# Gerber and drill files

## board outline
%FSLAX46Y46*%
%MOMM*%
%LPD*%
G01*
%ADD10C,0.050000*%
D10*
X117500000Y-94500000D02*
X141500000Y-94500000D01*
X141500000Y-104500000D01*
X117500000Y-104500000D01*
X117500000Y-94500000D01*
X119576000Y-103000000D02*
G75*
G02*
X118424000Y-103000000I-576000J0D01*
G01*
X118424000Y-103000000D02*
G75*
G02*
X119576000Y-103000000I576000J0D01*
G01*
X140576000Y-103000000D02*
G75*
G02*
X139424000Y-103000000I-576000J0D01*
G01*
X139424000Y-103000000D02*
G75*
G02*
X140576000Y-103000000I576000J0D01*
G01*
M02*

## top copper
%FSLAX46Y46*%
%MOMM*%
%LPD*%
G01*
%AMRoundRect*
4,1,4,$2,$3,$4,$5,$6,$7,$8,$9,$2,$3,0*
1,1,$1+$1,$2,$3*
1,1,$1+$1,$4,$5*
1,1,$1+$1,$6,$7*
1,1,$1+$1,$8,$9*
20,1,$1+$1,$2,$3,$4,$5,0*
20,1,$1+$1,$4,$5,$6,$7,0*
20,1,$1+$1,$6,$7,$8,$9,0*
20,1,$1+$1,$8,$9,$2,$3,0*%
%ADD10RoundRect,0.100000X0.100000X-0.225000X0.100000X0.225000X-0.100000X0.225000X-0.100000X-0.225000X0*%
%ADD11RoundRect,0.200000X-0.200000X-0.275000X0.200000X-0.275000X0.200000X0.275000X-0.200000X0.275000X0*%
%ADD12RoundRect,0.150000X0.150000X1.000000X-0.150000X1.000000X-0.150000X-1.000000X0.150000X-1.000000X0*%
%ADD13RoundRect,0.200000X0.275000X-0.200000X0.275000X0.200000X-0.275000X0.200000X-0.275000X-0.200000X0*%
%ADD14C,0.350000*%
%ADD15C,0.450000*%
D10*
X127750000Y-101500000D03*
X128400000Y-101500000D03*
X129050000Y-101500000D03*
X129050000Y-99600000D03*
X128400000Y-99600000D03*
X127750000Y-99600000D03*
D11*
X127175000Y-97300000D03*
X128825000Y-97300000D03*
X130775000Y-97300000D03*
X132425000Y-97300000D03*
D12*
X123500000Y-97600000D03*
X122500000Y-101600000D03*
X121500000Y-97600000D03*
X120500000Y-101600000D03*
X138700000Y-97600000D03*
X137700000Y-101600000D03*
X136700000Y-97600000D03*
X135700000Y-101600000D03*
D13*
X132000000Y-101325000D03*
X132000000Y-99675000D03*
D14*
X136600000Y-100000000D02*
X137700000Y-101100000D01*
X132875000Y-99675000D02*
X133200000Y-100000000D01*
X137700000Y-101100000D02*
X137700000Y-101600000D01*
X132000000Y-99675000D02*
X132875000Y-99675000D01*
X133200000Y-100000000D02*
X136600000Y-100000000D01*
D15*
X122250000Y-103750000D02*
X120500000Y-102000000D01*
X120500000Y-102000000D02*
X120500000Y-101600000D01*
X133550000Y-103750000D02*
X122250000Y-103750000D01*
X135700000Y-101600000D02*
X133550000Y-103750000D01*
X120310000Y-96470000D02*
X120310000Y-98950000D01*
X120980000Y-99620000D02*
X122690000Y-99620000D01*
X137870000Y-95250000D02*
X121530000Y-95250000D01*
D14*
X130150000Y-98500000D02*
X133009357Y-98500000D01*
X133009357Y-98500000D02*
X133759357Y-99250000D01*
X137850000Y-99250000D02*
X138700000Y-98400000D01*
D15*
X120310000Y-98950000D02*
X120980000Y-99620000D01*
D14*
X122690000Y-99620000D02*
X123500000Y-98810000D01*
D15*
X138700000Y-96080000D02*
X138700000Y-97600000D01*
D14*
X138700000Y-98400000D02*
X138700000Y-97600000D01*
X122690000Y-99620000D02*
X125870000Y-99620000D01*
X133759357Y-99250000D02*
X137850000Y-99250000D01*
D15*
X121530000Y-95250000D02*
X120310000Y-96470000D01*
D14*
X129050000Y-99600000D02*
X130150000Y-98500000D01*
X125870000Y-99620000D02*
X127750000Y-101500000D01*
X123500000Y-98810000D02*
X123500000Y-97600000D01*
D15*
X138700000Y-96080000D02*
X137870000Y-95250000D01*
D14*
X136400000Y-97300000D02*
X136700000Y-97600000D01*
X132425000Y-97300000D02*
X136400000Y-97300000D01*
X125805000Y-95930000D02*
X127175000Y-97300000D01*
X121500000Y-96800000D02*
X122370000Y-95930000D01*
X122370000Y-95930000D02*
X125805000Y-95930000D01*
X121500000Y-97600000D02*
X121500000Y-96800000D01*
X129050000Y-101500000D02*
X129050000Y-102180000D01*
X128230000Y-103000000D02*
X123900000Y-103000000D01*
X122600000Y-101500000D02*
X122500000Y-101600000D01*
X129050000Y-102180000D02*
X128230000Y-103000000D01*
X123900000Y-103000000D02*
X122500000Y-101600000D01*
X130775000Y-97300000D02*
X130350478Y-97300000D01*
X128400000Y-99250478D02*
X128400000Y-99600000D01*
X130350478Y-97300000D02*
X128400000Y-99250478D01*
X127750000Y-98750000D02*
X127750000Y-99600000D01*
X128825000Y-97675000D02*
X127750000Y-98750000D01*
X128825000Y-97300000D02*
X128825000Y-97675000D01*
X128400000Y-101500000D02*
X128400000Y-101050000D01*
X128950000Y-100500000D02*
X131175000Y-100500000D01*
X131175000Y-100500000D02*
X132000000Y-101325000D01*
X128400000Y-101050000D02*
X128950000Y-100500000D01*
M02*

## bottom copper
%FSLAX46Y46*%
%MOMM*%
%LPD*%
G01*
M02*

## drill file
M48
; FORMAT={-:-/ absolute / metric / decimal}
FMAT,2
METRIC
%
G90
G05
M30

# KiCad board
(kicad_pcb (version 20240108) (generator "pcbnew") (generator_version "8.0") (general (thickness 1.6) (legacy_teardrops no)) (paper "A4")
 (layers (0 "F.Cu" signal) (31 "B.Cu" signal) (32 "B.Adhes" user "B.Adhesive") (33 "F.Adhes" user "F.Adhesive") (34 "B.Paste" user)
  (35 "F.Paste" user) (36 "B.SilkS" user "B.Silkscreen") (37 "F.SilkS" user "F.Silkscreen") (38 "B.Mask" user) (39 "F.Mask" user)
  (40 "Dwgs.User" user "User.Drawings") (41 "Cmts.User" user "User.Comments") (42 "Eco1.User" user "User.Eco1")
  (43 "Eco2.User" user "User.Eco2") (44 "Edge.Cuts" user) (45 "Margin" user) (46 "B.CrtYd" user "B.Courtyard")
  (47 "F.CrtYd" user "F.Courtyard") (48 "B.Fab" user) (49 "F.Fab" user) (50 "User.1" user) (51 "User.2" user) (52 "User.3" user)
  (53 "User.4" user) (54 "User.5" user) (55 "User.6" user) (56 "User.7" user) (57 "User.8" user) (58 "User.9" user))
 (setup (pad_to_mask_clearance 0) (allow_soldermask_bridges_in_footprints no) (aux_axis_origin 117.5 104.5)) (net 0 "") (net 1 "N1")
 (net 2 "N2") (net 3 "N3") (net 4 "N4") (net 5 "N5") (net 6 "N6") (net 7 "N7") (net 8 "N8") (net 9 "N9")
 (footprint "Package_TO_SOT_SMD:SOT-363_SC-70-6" (layer "F.Cu") (at 128.4 100.55 90)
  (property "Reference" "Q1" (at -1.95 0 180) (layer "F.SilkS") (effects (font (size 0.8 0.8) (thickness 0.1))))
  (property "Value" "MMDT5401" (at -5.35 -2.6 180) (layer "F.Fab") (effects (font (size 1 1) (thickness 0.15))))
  (pad "1" smd roundrect (at -0.95 -0.65 90) (size 0.65 0.4) (layers "F.Cu" "F.Paste" "F.Mask") (roundrect_rratio 0.25) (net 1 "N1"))
  (pad "2" smd roundrect (at -0.95 0 90) (size 0.65 0.4) (layers "F.Cu" "F.Paste" "F.Mask") (roundrect_rratio 0.25) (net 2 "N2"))
  (pad "3" smd roundrect (at -0.95 0.65 90) (size 0.65 0.4) (layers "F.Cu" "F.Paste" "F.Mask") (roundrect_rratio 0.25) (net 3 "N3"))
  (pad "4" smd roundrect (at 0.95 0.65 90) (size 0.65 0.4) (layers "F.Cu" "F.Paste" "F.Mask") (roundrect_rratio 0.25) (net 1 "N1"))
  (pad "5" smd roundrect (at 0.95 0 90) (size 0.65 0.4) (layers "F.Cu" "F.Paste" "F.Mask") (roundrect_rratio 0.25) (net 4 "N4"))
  (pad "6" smd roundrect (at 0.95 -0.65 90) (size 0.65 0.4) (layers "F.Cu" "F.Paste" "F.Mask") (roundrect_rratio 0.25) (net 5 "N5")))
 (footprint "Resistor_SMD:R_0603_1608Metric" (layer "F.Cu") (at 128 97.3)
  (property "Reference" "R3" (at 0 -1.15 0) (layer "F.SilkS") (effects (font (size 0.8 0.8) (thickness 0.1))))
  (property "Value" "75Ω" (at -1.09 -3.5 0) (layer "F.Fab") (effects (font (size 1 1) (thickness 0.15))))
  (pad "1" smd roundrect (at -0.825 0) (size 0.8 0.95) (layers "F.Cu" "F.Paste" "F.Mask") (roundrect_rratio 0.25) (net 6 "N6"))
  (pad "2" smd roundrect (at 0.825 0) (size 0.8 0.95) (layers "F.Cu" "F.Paste" "F.Mask") (roundrect_rratio 0.25) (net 5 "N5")))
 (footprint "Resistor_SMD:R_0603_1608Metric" (layer "F.Cu") (at 131.6 97.3)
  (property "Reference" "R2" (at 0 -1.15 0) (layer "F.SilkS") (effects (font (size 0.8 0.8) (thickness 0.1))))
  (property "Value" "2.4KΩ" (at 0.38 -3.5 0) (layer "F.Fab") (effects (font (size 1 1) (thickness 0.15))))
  (pad "1" smd roundrect (at -0.825 0) (size 0.8 0.95) (layers "F.Cu" "F.Paste" "F.Mask") (roundrect_rratio 0.25) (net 4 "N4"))
  (pad "2" smd roundrect (at 0.825 0) (size 0.8 0.95) (layers "F.Cu" "F.Paste" "F.Mask") (roundrect_rratio 0.25) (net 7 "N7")))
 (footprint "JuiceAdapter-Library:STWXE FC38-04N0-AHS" (layer "F.Cu") (at 122 99.6 180)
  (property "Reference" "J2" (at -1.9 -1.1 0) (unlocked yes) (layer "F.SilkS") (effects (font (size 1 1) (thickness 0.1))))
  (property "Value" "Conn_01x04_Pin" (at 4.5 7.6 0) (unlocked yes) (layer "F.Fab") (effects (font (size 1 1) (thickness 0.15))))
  (pad "1" smd roundrect (at -1.5 2 180) (size 0.6 2.3) (layers "F.Cu" "F.Paste" "F.Mask") (roundrect_rratio 0.25) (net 1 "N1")
   (thermal_bridge_angle 45))
  (pad "2" smd roundrect (at -0.5 -2 180) (size 0.6 2.3) (layers "F.Cu" "F.Paste" "F.Mask") (roundrect_rratio 0.25) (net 3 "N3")
   (thermal_bridge_angle 45))
  (pad "3" smd roundrect (at 0.5 2 180) (size 0.6 2.3) (layers "F.Cu" "F.Paste" "F.Mask") (roundrect_rratio 0.25) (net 6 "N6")
   (thermal_bridge_angle 45))
  (pad "4" smd roundrect (at 1.5 -2 180) (size 0.6 2.3) (layers "F.Cu" "F.Paste" "F.Mask") (roundrect_rratio 0.25) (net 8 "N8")
   (thermal_bridge_angle 45)))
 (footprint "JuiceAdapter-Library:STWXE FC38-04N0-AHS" (layer "F.Cu") (at 137.2 99.6 180)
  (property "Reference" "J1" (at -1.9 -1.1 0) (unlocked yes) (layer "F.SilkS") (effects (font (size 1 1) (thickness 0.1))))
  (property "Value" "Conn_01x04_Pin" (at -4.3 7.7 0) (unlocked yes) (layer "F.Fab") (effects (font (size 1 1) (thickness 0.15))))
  (pad "1" smd roundrect (at -1.5 2 180) (size 0.6 2.3) (layers "F.Cu" "F.Paste" "F.Mask") (roundrect_rratio 0.25) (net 1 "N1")
   (thermal_bridge_angle 45))
  (pad "2" smd roundrect (at -0.5 -2 180) (size 0.6 2.3) (layers "F.Cu" "F.Paste" "F.Mask") (roundrect_rratio 0.25) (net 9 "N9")
   (thermal_bridge_angle 45))
  (pad "3" smd roundrect (at 0.5 2 180) (size 0.6 2.3) (layers "F.Cu" "F.Paste" "F.Mask") (roundrect_rratio 0.25) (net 7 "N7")
   (thermal_bridge_angle 45))
  (pad "4" smd roundrect (at 1.5 -2 180) (size 0.6 2.3) (layers "F.Cu" "F.Paste" "F.Mask") (roundrect_rratio 0.25) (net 8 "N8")
   (thermal_bridge_angle 45)))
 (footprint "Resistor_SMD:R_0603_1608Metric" (layer "F.Cu") (at 132 100.5 90)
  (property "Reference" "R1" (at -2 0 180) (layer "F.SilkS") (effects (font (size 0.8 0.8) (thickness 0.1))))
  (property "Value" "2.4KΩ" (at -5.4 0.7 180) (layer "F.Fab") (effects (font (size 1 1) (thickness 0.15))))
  (pad "1" smd roundrect (at -0.825 0 90) (size 0.8 0.95) (layers "F.Cu" "F.Paste" "F.Mask") (roundrect_rratio 0.25) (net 2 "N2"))
  (pad "2" smd roundrect (at 0.825 0 90) (size 0.8 0.95) (layers "F.Cu" "F.Paste" "F.Mask") (roundrect_rratio 0.25) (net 9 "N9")))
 (gr_rect (start 117.5 94.5) (end 141.5 104.5) (stroke (width 0.05) (type default)) (fill none) (layer "Edge.Cuts"))
 (gr_circle (center 119 103) (end 119.576 103) (stroke (width 0.05) (type default)) (fill none) (layer "Edge.Cuts"))
 (gr_circle (center 140 103) (end 140.576 103) (stroke (width 0.05) (type default)) (fill none) (layer "Edge.Cuts"))
 (segment (start 136.6 100) (end 137.7 101.1) (width 0.35) (layer "F.Cu") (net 9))
 (segment (start 132.875 99.675) (end 133.2 100) (width 0.35) (layer "F.Cu") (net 9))
 (segment (start 137.7 101.1) (end 137.7 101.6) (width 0.35) (layer "F.Cu") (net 9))
 (segment (start 132 99.675) (end 132.875 99.675) (width 0.35) (layer "F.Cu") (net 9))
 (segment (start 133.2 100) (end 136.6 100) (width 0.35) (layer "F.Cu") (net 9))
 (segment (start 122.25 103.75) (end 120.5 102) (width 0.45) (layer "F.Cu") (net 8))
 (segment (start 120.5 102) (end 120.5 101.6) (width 0.45) (layer "F.Cu") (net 8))
 (segment (start 133.55 103.75) (end 122.25 103.75) (width 0.45) (layer "F.Cu") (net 8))
 (segment (start 135.7 101.6) (end 133.55 103.75) (width 0.45) (layer "F.Cu") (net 8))
 (segment (start 120.31 96.47) (end 120.31 98.95) (width 0.45) (layer "F.Cu") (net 1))
 (segment (start 120.98 99.62) (end 122.69 99.62) (width 0.45) (layer "F.Cu") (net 1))
 (segment (start 137.87 95.25) (end 121.53 95.25) (width 0.45) (layer "F.Cu") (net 1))
 (segment (start 130.15 98.5) (end 133.009357 98.5) (width 0.35) (layer "F.Cu") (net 1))
 (segment (start 133.009357 98.5) (end 133.759357 99.25) (width 0.35) (layer "F.Cu") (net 1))
 (segment (start 137.85 99.25) (end 138.7 98.4) (width 0.35) (layer "F.Cu") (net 1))
 (segment (start 120.31 98.95) (end 120.98 99.62) (width 0.45) (layer "F.Cu") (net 1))
 (segment (start 122.69 99.62) (end 123.5 98.81) (width 0.35) (layer "F.Cu") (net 1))
 (segment (start 138.7 96.08) (end 138.7 97.6) (width 0.45) (layer "F.Cu") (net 1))
 (segment (start 138.7 98.4) (end 138.7 97.6) (width 0.35) (layer "F.Cu") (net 1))
 (segment (start 122.69 99.62) (end 125.87 99.62) (width 0.35) (layer "F.Cu") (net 1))
 (segment (start 133.759357 99.25) (end 137.85 99.25) (width 0.35) (layer "F.Cu") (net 1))
 (segment (start 121.53 95.25) (end 120.31 96.47) (width 0.45) (layer "F.Cu") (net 1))
 (segment (start 129.05 99.6) (end 130.15 98.5) (width 0.35) (layer "F.Cu") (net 1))
 (segment (start 125.87 99.62) (end 127.75 101.5) (width 0.35) (layer "F.Cu") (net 1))
 (segment (start 123.5 98.81) (end 123.5 97.6) (width 0.35) (layer "F.Cu") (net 1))
 (segment (start 138.7 96.08) (end 137.87 95.25) (width 0.45) (layer "F.Cu") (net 1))
 (segment (start 136.4 97.3) (end 136.7 97.6) (width 0.35) (layer "F.Cu") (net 7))
 (segment (start 132.425 97.3) (end 136.4 97.3) (width 0.35) (layer "F.Cu") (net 7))
 (segment (start 125.805 95.93) (end 127.175 97.3) (width 0.35) (layer "F.Cu") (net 6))
 (segment (start 121.5 96.8) (end 122.37 95.93) (width 0.35) (layer "F.Cu") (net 6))
 (segment (start 122.37 95.93) (end 125.805 95.93) (width 0.35) (layer "F.Cu") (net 6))
 (segment (start 121.5 97.6) (end 121.5 96.8) (width 0.35) (layer "F.Cu") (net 6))
 (segment (start 129.05 101.5) (end 129.05 102.18) (width 0.35) (layer "F.Cu") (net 3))
 (segment (start 128.23 103) (end 123.9 103) (width 0.35) (layer "F.Cu") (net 3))
 (segment (start 122.6 101.5) (end 122.5 101.6) (width 0.35) (layer "F.Cu") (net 3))
 (segment (start 129.05 102.18) (end 128.23 103) (width 0.35) (layer "F.Cu") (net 3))
 (segment (start 123.9 103) (end 122.5 101.6) (width 0.35) (layer "F.Cu") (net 3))
 (segment (start 130.775 97.3) (end 130.350478 97.3) (width 0.35) (layer "F.Cu") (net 4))
 (segment (start 128.4 99.250478) (end 128.4 99.6) (width 0.35) (layer "F.Cu") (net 4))
 (segment (start 130.350478 97.3) (end 128.4 99.250478) (width 0.35) (layer "F.Cu") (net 4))
 (segment (start 127.75 98.75) (end 127.75 99.6) (width 0.35) (layer "F.Cu") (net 5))
 (segment (start 128.825 97.675) (end 127.75 98.75) (width 0.35) (layer "F.Cu") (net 5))
 (segment (start 128.825 97.3) (end 128.825 97.675) (width 0.35) (layer "F.Cu") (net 5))
 (segment (start 128.4 101.5) (end 128.4 101.05) (width 0.35) (layer "F.Cu") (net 2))
 (segment (start 128.95 100.5) (end 131.175 100.5) (width 0.35) (layer "F.Cu") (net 2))
 (segment (start 131.175 100.5) (end 132 101.325) (width 0.35) (layer "F.Cu") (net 2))
 (segment (start 128.4 101.05) (end 128.95 100.5) (width 0.35) (layer "F.Cu") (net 2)))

